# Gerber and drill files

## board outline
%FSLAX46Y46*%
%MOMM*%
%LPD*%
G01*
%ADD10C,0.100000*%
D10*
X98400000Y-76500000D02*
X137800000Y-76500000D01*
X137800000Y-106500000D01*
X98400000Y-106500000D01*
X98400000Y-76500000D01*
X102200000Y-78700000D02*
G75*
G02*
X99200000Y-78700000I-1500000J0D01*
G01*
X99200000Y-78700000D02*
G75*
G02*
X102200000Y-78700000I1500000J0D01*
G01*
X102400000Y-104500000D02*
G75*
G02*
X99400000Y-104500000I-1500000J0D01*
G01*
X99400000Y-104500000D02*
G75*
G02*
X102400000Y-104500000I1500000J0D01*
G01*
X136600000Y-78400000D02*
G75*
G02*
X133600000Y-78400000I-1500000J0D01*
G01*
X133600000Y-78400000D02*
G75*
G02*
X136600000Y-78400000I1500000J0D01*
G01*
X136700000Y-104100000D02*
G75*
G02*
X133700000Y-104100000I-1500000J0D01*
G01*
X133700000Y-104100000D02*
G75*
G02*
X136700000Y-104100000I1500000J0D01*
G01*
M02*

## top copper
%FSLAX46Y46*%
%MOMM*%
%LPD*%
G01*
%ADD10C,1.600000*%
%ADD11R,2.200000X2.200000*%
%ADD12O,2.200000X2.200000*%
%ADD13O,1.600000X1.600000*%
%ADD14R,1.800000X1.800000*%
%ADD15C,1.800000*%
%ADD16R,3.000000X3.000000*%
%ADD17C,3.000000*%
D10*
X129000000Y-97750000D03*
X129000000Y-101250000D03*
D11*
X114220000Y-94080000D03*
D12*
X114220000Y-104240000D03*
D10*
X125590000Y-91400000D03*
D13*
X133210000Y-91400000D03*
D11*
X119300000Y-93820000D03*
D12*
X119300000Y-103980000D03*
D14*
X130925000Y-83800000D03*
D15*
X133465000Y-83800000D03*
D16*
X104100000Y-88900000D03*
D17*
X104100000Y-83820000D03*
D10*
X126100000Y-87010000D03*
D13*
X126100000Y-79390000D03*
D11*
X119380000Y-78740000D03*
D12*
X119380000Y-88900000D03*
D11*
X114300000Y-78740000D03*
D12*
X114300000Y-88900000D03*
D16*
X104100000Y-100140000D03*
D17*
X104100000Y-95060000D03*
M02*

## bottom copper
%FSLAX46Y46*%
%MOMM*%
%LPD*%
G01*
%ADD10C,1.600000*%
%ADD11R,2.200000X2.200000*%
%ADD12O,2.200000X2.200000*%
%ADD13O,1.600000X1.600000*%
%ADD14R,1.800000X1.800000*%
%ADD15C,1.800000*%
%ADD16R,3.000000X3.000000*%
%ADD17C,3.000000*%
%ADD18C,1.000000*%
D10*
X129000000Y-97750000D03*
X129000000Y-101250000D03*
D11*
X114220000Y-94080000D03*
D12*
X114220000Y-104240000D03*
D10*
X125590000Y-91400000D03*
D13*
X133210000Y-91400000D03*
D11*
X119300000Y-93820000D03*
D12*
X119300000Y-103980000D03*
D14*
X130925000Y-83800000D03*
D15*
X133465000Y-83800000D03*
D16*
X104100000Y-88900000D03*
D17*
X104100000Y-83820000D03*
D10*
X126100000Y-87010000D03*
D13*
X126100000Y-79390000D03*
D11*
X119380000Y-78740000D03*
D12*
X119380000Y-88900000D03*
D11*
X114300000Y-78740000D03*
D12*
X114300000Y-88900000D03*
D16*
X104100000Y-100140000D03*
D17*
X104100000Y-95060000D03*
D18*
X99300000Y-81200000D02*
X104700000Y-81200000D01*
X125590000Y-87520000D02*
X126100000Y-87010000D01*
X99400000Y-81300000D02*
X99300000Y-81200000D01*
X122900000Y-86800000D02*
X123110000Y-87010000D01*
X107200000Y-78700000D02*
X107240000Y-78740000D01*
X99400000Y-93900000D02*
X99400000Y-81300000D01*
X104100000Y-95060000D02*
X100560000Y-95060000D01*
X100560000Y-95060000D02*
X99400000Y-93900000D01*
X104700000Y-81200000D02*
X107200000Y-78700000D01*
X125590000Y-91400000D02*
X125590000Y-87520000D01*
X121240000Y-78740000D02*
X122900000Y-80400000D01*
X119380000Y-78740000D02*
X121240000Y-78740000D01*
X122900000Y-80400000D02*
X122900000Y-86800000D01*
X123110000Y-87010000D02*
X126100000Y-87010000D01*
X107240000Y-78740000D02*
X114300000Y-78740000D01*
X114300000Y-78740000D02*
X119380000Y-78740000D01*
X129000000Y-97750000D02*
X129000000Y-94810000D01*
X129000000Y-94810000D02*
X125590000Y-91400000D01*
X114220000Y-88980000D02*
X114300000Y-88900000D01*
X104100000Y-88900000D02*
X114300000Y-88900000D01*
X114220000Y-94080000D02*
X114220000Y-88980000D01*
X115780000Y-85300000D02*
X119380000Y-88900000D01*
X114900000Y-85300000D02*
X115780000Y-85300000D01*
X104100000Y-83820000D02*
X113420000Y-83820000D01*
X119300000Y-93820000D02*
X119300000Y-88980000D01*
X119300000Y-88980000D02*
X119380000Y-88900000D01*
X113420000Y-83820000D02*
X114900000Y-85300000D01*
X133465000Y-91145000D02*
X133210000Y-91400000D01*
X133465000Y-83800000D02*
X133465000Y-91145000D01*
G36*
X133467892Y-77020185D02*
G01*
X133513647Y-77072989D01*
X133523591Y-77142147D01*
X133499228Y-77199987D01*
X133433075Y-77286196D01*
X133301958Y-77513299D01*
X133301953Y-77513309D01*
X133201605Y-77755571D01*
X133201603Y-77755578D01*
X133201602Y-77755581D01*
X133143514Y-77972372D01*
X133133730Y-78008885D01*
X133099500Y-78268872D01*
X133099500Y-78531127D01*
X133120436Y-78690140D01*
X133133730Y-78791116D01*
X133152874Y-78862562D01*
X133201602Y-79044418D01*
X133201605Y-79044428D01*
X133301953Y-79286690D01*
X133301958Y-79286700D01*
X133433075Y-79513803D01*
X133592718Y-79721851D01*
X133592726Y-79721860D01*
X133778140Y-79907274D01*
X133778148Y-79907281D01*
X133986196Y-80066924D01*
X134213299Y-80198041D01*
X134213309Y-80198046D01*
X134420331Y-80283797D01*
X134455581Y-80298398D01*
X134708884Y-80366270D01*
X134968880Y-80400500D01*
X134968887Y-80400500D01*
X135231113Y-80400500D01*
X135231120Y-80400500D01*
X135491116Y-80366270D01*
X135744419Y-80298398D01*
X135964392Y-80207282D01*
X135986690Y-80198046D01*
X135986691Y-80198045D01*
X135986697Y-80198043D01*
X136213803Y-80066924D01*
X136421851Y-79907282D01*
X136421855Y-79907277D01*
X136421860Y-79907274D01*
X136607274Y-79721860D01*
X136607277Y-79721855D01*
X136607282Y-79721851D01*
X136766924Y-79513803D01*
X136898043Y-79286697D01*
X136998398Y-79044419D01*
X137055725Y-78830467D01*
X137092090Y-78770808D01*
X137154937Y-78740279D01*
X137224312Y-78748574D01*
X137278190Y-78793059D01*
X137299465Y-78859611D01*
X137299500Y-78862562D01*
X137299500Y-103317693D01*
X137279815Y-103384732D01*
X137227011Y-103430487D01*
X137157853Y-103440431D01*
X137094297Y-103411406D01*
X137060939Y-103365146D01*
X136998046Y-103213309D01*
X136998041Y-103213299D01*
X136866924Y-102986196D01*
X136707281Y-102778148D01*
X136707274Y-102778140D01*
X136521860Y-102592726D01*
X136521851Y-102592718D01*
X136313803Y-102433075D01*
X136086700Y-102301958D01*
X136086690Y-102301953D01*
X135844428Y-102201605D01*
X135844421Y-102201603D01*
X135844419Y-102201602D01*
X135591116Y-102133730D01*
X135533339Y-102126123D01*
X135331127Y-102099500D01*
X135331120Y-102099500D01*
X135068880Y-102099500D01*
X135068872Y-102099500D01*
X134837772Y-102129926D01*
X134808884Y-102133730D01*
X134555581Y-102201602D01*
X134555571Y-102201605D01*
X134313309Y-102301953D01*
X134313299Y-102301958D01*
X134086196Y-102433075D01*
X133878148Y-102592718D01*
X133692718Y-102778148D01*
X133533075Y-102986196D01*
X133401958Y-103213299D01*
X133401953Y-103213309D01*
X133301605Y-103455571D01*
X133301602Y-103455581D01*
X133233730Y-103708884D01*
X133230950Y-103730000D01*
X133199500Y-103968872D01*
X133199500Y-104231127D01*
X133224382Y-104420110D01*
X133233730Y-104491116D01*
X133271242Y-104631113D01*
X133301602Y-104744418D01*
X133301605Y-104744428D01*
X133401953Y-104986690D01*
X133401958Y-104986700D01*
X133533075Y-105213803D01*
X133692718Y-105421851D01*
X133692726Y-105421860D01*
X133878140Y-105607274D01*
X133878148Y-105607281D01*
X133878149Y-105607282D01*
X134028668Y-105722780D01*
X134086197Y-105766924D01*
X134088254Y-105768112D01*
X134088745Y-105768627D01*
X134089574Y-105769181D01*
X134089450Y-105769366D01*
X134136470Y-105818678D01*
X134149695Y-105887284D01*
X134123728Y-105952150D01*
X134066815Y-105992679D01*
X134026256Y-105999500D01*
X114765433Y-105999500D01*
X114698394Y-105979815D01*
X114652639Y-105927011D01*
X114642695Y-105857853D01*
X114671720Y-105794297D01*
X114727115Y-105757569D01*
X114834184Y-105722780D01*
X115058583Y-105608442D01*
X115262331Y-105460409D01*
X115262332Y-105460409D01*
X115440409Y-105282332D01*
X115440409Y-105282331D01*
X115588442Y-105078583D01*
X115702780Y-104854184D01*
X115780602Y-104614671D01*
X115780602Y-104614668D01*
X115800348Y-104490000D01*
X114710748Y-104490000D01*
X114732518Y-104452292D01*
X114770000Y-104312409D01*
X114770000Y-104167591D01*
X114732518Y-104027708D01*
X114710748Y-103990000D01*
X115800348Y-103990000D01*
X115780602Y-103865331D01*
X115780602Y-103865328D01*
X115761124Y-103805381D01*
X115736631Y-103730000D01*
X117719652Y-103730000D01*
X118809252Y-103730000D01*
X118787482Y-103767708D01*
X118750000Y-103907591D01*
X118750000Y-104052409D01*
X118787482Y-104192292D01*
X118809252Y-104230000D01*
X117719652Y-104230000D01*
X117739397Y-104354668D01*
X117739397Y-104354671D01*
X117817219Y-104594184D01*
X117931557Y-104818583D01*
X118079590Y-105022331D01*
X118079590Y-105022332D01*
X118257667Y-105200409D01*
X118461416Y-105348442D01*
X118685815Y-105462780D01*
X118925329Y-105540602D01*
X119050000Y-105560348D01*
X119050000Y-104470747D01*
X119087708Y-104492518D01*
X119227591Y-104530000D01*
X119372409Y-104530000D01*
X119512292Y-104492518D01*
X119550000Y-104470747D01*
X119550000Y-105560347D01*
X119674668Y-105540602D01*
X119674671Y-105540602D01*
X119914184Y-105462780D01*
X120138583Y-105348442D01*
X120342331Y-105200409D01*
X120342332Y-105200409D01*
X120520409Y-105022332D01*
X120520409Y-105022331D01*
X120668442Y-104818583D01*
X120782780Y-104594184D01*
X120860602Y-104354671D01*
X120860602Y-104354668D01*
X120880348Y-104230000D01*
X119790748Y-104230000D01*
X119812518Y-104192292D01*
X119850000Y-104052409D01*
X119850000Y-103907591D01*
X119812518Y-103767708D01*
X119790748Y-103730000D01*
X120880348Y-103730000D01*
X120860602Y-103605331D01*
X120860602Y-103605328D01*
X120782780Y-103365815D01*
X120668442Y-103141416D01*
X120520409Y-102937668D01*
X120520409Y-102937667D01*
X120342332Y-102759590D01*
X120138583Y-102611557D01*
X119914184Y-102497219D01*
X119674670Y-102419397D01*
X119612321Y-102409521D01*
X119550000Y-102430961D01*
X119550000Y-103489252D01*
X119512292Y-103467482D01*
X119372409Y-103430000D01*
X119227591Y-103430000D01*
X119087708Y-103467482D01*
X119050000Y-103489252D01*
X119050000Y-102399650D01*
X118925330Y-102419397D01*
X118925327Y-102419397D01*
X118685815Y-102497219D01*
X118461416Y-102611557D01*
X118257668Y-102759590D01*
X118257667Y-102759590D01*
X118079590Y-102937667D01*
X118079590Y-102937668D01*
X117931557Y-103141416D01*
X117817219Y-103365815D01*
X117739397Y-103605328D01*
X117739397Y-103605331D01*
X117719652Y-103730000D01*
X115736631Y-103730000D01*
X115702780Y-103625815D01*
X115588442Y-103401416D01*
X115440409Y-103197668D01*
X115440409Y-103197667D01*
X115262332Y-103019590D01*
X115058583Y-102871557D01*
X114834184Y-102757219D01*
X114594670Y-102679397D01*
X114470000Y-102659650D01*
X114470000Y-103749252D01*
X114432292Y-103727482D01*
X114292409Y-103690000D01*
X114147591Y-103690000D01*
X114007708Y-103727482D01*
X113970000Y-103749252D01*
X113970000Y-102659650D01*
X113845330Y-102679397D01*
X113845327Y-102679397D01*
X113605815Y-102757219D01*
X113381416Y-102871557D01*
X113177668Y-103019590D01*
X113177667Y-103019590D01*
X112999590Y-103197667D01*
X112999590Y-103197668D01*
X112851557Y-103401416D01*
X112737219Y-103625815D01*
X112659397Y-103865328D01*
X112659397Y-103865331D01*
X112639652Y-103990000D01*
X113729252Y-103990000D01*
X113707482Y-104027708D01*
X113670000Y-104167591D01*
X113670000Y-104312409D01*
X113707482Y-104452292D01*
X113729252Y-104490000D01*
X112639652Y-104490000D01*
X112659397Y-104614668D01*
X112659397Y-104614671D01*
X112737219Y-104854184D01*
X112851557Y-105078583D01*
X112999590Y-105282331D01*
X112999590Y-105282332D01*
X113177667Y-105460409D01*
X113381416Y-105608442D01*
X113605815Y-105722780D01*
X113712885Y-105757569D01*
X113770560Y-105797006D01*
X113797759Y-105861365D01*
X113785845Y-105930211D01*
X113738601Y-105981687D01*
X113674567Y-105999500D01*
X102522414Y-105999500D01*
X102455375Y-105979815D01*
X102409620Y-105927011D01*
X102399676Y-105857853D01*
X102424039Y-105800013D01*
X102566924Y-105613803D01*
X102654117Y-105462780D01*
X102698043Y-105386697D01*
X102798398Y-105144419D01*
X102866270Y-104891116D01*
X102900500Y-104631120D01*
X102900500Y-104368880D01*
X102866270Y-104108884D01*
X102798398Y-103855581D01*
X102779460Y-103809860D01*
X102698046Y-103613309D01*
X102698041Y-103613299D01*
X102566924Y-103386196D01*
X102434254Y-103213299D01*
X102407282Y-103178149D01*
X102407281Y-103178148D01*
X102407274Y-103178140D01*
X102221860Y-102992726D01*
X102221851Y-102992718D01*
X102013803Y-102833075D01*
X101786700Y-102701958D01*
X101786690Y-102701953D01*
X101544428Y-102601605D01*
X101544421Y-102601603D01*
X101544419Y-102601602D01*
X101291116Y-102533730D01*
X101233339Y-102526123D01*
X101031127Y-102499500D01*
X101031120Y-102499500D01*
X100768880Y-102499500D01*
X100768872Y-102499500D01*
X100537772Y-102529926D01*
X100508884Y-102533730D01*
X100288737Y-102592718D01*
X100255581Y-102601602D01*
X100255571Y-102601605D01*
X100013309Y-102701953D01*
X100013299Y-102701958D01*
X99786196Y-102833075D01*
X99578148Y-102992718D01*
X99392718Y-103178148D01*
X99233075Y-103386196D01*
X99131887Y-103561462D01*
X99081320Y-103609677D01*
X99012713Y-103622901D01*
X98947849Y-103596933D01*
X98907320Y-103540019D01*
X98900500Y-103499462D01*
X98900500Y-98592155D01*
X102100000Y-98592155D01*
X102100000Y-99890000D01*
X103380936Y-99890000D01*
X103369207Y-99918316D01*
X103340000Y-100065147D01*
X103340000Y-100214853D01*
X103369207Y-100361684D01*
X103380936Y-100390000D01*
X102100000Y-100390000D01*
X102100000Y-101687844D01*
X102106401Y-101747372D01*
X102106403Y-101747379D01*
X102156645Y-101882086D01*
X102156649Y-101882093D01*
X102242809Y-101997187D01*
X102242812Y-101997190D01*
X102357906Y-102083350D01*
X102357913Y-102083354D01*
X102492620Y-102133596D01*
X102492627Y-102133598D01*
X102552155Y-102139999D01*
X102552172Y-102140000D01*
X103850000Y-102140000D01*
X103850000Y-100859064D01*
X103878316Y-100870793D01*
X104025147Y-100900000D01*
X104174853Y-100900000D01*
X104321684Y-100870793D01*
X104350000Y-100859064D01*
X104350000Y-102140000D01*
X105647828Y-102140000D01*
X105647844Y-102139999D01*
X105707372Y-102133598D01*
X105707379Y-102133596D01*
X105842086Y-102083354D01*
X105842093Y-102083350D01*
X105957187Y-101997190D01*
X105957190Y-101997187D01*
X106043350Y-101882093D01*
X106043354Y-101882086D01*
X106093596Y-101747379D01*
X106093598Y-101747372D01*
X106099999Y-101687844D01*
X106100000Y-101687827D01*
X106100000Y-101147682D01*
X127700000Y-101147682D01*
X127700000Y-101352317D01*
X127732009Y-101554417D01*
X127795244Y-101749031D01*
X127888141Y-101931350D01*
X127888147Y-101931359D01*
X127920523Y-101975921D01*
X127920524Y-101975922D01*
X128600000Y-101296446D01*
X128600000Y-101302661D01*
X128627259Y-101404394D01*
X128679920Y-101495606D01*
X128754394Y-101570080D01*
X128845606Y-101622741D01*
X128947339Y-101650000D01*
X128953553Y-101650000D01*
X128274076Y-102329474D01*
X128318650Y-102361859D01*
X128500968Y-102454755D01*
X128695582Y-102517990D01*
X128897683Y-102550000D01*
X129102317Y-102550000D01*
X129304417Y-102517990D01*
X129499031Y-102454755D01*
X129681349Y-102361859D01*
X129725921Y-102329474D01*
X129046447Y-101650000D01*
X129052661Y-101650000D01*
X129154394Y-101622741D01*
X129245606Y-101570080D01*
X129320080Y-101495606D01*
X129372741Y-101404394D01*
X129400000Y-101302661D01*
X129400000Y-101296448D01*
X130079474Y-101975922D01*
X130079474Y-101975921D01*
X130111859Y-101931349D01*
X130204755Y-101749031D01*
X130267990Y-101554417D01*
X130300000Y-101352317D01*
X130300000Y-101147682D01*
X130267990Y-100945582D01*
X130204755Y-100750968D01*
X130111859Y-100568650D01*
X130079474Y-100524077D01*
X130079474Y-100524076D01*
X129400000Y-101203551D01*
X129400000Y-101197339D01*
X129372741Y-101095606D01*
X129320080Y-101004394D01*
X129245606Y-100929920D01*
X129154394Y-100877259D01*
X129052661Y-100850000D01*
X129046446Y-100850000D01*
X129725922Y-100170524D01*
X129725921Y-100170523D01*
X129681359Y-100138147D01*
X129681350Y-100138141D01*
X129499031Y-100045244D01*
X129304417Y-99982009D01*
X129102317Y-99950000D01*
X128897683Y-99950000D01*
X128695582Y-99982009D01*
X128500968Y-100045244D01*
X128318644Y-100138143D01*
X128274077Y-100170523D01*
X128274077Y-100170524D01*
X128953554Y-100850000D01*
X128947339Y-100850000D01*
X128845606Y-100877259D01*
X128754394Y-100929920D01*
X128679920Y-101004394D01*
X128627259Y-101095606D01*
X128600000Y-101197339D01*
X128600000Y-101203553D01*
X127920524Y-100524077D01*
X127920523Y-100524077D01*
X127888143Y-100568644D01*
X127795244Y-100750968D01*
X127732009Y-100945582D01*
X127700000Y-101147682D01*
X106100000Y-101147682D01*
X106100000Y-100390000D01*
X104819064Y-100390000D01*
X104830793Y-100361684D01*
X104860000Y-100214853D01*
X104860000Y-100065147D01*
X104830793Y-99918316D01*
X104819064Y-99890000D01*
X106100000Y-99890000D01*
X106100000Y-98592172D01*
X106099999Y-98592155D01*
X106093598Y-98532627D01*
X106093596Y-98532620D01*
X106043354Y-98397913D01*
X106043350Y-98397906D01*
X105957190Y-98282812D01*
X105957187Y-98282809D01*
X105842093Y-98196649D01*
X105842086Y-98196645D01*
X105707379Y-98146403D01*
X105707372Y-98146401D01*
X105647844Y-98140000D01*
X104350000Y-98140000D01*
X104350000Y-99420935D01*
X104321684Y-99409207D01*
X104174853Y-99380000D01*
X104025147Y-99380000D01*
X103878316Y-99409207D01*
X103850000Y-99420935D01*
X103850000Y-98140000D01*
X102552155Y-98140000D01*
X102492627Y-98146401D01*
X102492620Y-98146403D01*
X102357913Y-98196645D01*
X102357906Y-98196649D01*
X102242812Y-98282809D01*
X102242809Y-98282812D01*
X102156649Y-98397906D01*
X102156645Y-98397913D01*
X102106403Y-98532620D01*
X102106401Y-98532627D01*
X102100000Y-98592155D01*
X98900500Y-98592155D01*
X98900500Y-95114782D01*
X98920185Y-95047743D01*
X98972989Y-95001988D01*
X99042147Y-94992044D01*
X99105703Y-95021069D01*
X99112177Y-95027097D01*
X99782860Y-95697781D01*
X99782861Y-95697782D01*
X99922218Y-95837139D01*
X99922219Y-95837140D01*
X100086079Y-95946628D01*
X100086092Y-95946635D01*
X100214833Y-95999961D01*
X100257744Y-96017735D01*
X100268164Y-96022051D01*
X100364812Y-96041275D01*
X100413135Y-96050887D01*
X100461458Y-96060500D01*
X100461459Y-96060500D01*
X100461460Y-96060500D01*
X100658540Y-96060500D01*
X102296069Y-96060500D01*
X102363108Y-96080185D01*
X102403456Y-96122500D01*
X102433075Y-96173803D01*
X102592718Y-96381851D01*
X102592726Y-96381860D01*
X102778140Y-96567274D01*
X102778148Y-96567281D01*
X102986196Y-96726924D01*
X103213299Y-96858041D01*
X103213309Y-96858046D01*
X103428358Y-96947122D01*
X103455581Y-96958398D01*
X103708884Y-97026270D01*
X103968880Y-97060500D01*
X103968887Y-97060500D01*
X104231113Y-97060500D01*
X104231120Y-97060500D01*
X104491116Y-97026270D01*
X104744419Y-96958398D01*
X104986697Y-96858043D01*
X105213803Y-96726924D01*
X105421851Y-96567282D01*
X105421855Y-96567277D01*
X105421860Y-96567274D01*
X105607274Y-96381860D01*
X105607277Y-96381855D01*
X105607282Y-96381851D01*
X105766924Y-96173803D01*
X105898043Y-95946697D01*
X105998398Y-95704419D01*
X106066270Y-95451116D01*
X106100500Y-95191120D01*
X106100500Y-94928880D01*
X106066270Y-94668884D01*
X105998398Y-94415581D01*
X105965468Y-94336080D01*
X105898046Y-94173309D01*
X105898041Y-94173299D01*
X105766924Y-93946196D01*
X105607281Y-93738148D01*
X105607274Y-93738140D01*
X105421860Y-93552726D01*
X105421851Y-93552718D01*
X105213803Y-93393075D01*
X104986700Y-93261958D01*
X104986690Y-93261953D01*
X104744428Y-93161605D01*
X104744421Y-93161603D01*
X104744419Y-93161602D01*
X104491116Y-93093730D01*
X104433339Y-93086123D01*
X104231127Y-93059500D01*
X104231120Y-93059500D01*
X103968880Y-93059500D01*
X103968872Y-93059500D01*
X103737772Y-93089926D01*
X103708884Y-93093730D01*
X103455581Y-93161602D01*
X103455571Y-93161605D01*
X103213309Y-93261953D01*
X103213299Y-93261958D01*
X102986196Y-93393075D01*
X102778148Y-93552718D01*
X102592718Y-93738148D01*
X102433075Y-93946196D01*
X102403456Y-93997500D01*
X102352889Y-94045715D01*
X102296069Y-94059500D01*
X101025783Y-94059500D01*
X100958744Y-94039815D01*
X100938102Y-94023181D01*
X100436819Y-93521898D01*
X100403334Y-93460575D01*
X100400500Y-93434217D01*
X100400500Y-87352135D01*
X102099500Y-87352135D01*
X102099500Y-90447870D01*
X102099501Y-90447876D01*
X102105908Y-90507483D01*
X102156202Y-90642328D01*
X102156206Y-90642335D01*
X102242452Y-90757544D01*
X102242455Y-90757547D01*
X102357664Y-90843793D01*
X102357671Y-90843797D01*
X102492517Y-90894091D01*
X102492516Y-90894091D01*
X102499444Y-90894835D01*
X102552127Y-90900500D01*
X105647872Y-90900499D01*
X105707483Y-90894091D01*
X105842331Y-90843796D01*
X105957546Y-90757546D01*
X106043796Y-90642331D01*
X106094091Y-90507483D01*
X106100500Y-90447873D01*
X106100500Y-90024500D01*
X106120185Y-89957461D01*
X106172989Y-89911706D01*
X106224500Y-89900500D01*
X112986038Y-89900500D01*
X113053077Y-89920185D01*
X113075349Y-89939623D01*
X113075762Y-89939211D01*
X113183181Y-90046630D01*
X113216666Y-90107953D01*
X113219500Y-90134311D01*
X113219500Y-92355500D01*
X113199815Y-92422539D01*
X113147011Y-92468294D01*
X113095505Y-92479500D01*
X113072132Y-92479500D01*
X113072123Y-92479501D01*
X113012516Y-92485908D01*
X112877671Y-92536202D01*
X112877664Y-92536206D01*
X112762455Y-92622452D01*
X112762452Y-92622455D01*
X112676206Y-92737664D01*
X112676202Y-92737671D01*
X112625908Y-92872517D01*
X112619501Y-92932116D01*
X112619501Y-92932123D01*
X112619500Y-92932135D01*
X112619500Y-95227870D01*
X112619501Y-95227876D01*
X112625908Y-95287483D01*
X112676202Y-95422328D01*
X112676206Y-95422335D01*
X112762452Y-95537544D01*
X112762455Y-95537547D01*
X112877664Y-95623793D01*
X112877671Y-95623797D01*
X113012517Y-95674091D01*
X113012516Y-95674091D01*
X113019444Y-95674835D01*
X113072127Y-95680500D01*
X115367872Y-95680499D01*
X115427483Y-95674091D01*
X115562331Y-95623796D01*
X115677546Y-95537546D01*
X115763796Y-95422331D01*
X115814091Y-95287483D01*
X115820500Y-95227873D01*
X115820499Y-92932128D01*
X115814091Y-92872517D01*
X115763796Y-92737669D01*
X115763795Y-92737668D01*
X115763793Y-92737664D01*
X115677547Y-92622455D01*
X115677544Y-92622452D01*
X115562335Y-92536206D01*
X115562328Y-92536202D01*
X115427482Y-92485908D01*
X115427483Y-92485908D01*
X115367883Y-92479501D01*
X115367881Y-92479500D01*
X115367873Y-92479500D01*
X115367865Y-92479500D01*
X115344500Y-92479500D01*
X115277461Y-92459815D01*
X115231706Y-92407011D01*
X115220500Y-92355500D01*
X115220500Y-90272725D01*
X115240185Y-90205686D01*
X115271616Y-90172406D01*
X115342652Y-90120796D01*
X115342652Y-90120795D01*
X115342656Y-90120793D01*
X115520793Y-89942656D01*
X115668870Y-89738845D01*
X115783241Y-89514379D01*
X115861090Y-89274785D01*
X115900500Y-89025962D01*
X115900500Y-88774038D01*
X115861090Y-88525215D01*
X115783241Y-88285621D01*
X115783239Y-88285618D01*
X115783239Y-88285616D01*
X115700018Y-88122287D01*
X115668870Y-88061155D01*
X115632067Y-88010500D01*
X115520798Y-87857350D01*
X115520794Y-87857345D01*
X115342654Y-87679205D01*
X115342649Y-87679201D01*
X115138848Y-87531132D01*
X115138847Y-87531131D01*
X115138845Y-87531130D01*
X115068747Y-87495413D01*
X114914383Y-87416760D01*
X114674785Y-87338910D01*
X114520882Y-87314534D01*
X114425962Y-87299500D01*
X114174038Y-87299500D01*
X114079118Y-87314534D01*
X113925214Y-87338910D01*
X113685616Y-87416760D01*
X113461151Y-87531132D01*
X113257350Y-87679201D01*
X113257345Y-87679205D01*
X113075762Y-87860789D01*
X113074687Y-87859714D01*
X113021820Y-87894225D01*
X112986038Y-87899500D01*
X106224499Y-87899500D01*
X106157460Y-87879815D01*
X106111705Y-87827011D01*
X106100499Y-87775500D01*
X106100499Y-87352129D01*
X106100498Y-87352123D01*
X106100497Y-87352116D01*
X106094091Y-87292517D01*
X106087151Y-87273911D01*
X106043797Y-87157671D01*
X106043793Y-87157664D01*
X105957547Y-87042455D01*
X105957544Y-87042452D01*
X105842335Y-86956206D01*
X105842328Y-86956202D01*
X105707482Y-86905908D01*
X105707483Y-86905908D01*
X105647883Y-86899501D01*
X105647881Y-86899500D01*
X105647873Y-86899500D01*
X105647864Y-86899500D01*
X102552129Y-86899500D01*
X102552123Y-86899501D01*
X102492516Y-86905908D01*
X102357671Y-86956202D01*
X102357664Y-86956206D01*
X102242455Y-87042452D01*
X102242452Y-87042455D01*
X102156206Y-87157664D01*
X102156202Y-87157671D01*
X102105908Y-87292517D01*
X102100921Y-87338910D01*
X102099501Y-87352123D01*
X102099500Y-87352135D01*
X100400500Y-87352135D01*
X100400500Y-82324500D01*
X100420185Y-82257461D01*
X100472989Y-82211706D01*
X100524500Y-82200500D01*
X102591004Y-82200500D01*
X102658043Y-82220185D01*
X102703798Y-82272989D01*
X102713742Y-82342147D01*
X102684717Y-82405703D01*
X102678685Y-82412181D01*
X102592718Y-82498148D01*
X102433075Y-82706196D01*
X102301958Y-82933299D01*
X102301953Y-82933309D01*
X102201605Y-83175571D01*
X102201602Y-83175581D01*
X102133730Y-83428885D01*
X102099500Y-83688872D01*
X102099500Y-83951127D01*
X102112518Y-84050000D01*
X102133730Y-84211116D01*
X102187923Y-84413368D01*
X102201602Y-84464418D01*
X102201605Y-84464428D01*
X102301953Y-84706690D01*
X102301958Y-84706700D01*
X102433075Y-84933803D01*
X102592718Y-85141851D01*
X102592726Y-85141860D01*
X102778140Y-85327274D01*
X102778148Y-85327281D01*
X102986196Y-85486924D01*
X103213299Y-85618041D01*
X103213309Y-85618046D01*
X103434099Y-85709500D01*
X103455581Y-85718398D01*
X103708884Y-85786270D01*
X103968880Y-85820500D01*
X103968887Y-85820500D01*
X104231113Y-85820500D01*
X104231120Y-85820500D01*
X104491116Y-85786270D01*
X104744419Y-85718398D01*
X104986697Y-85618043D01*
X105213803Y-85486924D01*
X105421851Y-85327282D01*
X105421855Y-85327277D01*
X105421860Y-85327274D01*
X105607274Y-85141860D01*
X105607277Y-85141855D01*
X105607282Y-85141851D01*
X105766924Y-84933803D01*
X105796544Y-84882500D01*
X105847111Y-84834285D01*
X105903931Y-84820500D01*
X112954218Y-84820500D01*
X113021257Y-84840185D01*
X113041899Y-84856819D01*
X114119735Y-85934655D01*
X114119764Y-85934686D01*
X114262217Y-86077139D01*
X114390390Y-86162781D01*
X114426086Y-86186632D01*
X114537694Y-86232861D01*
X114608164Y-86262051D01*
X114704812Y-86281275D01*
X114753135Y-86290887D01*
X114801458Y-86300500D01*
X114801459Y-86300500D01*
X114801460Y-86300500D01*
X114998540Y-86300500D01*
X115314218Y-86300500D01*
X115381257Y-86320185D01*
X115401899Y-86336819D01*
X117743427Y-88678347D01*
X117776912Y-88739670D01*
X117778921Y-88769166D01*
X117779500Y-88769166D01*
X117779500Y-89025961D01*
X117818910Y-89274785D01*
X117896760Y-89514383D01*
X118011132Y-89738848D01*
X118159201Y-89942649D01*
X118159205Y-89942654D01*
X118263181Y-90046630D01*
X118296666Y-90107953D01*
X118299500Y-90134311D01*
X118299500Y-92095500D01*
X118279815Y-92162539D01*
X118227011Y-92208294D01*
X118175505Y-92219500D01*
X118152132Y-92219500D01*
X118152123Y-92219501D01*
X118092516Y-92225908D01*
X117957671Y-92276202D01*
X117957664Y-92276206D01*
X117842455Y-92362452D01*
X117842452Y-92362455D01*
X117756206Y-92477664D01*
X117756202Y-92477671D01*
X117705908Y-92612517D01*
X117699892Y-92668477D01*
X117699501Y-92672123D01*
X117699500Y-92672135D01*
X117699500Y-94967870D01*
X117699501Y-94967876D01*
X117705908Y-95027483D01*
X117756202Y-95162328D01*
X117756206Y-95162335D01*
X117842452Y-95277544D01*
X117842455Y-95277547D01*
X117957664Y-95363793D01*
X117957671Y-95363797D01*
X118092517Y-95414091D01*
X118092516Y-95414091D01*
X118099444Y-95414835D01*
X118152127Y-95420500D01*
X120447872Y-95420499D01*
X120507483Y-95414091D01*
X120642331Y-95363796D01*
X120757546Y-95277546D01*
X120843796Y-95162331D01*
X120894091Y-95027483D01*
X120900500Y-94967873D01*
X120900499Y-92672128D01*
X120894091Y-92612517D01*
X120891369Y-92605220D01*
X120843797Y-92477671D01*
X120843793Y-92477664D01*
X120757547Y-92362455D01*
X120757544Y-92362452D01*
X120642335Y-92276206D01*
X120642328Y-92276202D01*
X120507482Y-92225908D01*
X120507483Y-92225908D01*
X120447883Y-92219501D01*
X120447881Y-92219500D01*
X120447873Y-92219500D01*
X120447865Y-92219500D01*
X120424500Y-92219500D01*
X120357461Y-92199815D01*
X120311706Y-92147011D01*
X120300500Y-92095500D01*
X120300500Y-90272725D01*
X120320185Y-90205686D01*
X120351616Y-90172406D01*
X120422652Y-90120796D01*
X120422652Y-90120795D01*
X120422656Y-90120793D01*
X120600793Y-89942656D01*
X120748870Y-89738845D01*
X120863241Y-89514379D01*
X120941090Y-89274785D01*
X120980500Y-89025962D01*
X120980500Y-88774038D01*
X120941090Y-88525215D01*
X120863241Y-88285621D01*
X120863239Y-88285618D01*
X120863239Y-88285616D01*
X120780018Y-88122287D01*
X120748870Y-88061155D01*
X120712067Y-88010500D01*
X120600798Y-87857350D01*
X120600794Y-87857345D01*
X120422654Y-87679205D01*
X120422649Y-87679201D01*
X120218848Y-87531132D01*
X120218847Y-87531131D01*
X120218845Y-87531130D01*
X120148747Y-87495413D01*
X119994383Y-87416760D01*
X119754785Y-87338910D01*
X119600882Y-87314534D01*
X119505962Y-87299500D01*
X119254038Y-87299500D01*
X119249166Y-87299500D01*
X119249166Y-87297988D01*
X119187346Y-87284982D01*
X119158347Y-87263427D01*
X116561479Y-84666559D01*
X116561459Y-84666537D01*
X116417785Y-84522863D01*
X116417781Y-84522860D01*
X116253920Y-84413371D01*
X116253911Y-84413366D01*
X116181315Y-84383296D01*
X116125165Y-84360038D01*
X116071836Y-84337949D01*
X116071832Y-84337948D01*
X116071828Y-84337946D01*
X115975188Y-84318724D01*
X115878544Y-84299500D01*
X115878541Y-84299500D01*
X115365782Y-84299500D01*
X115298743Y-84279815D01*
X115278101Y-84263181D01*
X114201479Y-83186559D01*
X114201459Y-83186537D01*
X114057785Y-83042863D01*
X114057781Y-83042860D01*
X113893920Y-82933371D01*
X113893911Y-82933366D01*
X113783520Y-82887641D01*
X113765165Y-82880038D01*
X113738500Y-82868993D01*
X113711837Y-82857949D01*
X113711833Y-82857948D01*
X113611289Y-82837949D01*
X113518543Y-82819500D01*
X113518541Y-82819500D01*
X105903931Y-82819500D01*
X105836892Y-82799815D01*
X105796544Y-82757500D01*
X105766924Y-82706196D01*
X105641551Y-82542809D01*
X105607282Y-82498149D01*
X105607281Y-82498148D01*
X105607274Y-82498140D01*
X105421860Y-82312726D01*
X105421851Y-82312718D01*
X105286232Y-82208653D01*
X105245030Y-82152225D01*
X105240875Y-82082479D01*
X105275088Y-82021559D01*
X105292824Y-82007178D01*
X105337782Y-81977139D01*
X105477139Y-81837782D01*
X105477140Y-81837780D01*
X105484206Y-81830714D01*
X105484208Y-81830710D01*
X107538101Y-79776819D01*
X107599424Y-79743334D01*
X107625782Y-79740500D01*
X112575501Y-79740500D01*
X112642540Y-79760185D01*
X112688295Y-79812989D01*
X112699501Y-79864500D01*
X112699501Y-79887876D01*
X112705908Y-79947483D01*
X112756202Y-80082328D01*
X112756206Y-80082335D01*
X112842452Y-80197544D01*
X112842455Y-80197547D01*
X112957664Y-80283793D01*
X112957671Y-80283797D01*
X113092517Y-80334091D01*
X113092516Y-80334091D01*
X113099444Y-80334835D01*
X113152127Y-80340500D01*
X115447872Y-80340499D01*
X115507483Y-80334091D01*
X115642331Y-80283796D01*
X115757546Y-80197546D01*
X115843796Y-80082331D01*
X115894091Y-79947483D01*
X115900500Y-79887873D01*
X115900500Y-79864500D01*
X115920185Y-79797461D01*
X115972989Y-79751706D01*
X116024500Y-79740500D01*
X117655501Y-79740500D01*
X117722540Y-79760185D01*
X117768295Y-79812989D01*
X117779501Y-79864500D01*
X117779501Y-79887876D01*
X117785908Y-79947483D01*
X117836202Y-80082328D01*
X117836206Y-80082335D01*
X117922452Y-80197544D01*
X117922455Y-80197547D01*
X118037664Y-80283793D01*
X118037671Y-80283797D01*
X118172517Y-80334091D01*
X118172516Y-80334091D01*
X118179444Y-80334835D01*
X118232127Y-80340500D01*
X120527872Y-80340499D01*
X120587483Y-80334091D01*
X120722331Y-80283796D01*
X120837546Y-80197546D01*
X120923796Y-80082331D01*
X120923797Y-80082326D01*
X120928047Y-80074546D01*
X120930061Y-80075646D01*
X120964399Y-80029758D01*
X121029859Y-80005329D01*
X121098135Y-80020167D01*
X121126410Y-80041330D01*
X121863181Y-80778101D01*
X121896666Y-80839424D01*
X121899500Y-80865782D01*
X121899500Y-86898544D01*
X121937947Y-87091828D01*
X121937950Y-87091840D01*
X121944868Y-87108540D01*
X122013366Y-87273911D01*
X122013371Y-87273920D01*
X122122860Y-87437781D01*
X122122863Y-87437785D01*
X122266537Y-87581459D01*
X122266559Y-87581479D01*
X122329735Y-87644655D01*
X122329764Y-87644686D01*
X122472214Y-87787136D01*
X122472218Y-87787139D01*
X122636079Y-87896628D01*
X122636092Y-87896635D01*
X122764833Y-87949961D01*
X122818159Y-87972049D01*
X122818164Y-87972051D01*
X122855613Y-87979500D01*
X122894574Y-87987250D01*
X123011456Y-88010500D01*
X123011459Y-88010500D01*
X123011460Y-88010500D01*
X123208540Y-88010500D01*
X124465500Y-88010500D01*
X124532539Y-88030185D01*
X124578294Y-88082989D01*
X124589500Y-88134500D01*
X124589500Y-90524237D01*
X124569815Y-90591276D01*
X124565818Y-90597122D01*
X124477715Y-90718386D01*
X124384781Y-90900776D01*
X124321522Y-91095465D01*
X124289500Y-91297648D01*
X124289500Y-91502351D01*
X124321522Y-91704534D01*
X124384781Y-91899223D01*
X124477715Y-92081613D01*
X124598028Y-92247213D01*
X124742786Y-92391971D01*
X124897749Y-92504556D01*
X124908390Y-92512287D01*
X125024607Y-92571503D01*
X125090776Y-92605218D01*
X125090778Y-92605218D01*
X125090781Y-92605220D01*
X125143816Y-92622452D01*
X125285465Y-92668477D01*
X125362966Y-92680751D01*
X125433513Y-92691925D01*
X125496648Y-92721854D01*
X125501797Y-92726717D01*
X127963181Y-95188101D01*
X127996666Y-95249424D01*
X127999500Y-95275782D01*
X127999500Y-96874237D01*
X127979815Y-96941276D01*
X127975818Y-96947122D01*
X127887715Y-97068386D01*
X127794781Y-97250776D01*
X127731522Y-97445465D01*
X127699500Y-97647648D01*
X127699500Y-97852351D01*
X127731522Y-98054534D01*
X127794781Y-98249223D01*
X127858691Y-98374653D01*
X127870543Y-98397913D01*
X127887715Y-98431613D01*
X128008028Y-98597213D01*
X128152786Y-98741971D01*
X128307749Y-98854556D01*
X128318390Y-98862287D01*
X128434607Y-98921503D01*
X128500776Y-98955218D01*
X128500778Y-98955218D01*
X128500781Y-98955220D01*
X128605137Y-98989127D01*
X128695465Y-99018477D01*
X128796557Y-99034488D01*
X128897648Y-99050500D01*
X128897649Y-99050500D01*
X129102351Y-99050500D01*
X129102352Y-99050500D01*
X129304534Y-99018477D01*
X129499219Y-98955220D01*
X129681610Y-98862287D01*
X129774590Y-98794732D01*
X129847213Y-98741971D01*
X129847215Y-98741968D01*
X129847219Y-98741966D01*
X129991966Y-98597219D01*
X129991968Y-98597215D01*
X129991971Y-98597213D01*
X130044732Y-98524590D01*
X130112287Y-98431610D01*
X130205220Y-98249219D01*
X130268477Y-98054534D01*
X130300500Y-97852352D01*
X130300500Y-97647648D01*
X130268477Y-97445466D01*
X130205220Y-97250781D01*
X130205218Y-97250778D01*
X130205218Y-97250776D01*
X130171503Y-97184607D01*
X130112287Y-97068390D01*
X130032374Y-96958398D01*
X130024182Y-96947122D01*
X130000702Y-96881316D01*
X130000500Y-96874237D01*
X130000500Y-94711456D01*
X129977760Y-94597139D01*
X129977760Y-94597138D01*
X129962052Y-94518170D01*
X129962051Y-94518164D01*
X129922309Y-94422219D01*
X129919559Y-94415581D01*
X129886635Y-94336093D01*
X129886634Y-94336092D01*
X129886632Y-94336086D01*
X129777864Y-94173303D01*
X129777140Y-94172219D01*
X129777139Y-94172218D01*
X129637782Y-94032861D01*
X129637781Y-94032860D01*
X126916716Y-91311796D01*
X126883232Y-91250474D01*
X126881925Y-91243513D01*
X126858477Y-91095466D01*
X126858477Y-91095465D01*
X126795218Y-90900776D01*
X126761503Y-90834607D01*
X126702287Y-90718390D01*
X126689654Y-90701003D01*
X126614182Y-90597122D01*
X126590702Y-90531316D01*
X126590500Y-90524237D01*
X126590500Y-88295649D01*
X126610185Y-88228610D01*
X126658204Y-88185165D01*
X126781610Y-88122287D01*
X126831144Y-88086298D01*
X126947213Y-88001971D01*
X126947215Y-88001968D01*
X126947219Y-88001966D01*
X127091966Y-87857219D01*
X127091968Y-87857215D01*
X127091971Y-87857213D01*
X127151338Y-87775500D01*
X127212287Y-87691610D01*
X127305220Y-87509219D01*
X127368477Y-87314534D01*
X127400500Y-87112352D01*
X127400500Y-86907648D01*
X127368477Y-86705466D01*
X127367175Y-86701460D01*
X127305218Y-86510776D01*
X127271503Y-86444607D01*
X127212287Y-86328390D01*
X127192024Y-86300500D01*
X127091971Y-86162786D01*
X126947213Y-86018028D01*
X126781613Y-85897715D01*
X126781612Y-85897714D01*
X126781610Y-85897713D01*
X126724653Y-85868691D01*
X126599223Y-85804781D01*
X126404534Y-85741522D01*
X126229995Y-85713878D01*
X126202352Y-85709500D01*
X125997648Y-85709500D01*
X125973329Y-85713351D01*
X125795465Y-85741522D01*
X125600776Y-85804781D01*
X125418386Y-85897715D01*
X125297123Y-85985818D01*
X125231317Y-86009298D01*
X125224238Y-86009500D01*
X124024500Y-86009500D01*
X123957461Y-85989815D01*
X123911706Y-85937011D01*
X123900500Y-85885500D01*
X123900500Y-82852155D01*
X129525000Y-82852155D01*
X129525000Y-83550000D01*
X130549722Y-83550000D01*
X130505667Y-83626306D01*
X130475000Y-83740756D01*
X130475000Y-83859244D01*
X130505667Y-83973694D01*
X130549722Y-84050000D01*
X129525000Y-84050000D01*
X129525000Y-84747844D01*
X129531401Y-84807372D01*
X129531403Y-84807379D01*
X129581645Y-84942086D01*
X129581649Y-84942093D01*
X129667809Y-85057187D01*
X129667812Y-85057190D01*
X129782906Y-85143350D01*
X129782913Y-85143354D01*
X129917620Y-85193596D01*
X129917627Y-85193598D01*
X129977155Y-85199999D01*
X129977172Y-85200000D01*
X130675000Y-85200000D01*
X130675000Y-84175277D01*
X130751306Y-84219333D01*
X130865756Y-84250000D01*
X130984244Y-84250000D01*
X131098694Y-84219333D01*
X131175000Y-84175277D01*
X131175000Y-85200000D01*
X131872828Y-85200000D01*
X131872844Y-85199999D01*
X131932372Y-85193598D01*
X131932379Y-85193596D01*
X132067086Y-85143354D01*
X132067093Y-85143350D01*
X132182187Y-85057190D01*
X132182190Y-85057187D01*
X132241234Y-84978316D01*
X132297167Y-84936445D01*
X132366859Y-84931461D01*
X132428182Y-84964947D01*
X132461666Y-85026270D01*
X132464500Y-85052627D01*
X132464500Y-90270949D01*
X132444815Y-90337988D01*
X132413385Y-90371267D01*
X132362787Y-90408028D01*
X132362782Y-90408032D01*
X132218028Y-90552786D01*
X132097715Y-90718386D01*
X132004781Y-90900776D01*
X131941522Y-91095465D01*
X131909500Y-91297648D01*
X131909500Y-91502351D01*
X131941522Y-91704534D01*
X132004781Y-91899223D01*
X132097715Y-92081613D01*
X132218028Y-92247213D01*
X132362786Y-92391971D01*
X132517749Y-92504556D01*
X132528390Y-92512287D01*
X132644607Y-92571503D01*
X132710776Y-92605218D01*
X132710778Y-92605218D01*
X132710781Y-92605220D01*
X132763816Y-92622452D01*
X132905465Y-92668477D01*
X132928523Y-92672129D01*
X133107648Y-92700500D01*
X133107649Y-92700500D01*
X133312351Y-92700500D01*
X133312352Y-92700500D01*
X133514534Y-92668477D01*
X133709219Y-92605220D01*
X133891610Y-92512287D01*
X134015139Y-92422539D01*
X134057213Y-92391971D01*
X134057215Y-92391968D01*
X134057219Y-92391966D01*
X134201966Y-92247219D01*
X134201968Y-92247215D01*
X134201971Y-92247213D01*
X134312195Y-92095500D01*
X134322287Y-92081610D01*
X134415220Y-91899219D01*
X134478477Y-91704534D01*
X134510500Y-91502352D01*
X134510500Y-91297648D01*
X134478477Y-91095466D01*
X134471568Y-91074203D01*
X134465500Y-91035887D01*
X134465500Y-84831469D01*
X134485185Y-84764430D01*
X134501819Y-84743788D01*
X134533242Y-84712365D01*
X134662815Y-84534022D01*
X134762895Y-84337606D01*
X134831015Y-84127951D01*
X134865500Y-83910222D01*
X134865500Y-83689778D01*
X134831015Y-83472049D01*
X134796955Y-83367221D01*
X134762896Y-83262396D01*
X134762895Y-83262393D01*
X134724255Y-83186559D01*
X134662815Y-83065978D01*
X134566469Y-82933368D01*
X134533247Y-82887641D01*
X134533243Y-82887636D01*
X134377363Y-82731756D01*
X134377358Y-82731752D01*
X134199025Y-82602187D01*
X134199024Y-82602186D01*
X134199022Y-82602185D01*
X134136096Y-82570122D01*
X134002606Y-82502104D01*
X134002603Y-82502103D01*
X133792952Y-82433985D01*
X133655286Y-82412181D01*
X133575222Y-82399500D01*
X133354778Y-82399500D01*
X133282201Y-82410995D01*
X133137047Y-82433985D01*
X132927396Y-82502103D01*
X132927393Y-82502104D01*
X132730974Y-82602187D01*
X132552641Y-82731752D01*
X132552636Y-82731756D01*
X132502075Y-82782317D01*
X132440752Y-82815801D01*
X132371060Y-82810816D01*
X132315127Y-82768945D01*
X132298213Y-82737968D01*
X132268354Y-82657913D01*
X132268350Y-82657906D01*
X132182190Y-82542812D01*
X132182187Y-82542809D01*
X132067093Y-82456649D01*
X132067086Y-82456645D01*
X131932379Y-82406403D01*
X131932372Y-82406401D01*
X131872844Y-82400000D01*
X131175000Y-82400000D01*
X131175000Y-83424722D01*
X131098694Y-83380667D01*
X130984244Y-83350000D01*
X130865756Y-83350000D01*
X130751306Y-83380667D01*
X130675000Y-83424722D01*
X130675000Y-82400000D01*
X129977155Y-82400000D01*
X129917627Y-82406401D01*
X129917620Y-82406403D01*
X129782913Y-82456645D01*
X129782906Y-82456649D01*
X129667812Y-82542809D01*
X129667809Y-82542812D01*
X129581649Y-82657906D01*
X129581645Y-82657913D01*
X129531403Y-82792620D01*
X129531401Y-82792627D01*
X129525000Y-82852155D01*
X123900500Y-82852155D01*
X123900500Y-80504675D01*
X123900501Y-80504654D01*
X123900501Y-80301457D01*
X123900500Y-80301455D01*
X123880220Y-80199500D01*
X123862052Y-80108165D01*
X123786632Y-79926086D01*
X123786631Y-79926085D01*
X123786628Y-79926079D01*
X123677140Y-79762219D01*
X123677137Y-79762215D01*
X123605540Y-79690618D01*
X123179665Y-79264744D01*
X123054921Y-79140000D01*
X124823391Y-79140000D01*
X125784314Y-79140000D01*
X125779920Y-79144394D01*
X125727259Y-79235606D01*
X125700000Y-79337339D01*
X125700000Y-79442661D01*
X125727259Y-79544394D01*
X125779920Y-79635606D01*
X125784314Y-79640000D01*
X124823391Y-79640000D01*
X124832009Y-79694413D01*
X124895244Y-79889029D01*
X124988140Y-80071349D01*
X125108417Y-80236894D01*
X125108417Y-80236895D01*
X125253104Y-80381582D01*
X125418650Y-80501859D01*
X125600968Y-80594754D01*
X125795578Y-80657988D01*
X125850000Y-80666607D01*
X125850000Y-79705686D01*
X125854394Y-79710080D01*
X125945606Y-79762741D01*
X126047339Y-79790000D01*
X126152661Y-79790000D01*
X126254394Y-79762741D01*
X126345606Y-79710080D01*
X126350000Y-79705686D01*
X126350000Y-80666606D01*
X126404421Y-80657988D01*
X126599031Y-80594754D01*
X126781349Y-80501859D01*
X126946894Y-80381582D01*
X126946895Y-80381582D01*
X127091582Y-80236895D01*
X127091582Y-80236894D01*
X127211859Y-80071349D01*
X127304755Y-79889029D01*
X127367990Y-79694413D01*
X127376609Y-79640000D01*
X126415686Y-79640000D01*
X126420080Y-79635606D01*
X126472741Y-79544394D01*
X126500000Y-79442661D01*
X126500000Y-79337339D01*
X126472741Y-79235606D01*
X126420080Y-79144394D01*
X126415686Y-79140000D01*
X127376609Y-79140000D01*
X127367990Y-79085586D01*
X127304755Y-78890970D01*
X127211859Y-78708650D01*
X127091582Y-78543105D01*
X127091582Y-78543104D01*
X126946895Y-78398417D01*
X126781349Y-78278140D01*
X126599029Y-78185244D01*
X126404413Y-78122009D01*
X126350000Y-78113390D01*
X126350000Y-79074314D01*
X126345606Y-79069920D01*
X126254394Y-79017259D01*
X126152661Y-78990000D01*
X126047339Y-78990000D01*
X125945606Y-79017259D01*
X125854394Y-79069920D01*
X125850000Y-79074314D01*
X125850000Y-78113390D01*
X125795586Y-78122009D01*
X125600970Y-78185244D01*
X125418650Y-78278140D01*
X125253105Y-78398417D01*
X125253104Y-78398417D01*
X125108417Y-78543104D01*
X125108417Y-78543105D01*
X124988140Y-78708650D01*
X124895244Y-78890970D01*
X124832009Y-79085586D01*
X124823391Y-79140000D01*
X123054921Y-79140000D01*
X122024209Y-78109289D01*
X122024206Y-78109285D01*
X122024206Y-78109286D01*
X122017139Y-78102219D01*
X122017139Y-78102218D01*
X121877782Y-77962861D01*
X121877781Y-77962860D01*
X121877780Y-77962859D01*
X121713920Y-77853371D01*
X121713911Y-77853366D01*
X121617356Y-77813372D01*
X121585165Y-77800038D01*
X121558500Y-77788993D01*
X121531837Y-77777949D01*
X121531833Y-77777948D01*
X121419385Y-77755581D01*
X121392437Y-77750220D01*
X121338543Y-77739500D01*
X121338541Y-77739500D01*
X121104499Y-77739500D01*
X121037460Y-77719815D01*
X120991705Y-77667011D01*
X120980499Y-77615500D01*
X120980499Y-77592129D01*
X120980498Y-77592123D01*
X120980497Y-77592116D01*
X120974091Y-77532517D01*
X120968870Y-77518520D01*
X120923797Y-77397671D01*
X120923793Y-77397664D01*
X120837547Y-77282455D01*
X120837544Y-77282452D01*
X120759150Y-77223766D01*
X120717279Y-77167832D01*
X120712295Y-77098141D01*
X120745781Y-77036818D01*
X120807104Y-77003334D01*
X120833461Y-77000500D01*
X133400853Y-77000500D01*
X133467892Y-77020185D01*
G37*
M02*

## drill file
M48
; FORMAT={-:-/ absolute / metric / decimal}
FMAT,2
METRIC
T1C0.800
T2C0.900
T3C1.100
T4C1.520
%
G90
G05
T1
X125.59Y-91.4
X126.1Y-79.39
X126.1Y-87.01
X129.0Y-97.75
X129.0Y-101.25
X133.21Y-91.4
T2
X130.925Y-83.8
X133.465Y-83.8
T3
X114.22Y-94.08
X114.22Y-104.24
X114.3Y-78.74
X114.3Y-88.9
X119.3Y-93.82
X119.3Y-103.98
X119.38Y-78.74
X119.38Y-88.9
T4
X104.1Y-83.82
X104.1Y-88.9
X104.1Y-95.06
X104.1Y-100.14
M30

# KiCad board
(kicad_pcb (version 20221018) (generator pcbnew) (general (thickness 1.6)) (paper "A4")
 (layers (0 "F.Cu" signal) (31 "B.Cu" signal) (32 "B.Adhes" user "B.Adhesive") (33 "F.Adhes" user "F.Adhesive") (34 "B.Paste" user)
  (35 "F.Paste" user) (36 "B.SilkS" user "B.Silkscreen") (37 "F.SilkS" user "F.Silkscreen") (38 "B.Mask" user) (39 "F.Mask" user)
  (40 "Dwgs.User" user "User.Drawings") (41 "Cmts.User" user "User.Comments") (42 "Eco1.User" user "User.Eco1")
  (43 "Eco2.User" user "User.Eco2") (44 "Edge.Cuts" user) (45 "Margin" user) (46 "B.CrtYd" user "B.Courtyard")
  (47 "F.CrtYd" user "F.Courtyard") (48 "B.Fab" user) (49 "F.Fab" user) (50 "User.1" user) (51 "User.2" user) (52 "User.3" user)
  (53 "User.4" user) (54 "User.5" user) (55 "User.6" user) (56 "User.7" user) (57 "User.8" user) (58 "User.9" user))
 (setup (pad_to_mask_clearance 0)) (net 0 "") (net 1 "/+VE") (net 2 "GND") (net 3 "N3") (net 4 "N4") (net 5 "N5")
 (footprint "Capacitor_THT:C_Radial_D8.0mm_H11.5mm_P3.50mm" (layer "F.Cu") (at 129 97.75 -90)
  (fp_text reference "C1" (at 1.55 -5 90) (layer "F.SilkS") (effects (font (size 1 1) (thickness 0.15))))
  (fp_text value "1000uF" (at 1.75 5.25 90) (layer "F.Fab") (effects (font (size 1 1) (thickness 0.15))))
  (pad "1" thru_hole circle (at 0 0 270) (size 1.6 1.6) (drill 0.8) (layers "*.Cu" "*.Mask") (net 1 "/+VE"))
  (pad "2" thru_hole circle (at 3.5 0 270) (size 1.6 1.6) (drill 0.8) (layers "*.Cu" "*.Mask") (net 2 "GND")))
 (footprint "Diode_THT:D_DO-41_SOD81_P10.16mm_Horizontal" (layer "F.Cu") (at 114.22 94.08 -90)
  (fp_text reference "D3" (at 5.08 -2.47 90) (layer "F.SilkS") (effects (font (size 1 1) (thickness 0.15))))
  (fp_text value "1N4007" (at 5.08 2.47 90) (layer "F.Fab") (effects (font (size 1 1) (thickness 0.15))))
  (pad "1" thru_hole rect (at 0 0 270) (size 2.2 2.2) (drill 1.1) (layers "*.Cu" "*.Mask") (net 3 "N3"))
  (pad "2" thru_hole oval (at 10.16 0 270) (size 2.2 2.2) (drill 1.1) (layers "*.Cu" "*.Mask") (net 2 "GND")))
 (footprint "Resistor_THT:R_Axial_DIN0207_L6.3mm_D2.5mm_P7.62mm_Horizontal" (layer "F.Cu") (at 125.59 91.4)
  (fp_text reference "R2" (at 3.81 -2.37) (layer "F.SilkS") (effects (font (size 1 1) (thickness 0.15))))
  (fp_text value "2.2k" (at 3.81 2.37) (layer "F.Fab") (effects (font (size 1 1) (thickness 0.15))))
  (pad "1" thru_hole circle (at 0 0) (size 1.6 1.6) (drill 0.8) (layers "*.Cu" "*.Mask") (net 1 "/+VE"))
  (pad "2" thru_hole oval (at 7.62 0) (size 1.6 1.6) (drill 0.8) (layers "*.Cu" "*.Mask") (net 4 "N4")))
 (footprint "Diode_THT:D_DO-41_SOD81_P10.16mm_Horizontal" (layer "F.Cu") (at 119.3 93.82 -90)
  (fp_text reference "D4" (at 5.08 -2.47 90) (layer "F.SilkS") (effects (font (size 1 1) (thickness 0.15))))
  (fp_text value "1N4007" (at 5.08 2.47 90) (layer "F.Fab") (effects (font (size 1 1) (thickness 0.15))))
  (pad "1" thru_hole rect (at 0 0 270) (size 2.2 2.2) (drill 1.1) (layers "*.Cu" "*.Mask") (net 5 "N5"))
  (pad "2" thru_hole oval (at 10.16 0 270) (size 2.2 2.2) (drill 1.1) (layers "*.Cu" "*.Mask") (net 2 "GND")))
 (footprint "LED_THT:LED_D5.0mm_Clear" (layer "F.Cu") (at 130.925 83.8)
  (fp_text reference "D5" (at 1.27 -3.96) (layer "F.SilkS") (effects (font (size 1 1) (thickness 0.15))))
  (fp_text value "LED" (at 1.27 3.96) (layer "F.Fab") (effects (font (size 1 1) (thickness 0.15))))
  (pad "1" thru_hole rect (at 0 0) (size 1.8 1.8) (drill 0.9) (layers "*.Cu" "*.Mask") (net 2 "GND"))
  (pad "2" thru_hole circle (at 2.54 0) (size 1.8 1.8) (drill 0.9) (layers "*.Cu" "*.Mask") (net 4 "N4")))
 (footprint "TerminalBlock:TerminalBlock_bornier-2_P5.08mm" (layer "F.Cu") (at 104.1 88.9 90)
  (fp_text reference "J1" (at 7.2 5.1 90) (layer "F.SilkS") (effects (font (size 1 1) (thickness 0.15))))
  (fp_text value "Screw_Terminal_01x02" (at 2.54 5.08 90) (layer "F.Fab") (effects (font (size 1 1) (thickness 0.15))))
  (pad "1" thru_hole rect (at 0 0 90) (size 3 3) (drill 1.52) (layers "*.Cu" "*.Mask") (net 3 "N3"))
  (pad "2" thru_hole circle (at 5.08 0 90) (size 3 3) (drill 1.52) (layers "*.Cu" "*.Mask") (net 5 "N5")))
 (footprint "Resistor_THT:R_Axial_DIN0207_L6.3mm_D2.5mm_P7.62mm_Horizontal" (layer "F.Cu") (at 126.1 87.01 90)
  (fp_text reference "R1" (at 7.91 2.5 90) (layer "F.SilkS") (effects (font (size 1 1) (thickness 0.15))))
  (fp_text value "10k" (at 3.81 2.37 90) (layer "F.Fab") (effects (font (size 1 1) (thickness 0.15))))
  (pad "1" thru_hole circle (at 0 0 90) (size 1.6 1.6) (drill 0.8) (layers "*.Cu" "*.Mask") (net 1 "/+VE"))
  (pad "2" thru_hole oval (at 7.62 0 90) (size 1.6 1.6) (drill 0.8) (layers "*.Cu" "*.Mask") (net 2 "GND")))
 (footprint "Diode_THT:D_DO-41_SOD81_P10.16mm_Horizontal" (layer "F.Cu") (at 119.38 78.74 -90)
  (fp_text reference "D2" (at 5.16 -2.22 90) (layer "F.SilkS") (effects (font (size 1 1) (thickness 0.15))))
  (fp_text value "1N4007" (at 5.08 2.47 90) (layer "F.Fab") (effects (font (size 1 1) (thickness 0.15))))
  (pad "1" thru_hole rect (at 0 0 270) (size 2.2 2.2) (drill 1.1) (layers "*.Cu" "*.Mask") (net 1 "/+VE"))
  (pad "2" thru_hole oval (at 10.16 0 270) (size 2.2 2.2) (drill 1.1) (layers "*.Cu" "*.Mask") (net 5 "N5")))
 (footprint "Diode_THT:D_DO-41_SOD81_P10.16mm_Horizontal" (layer "F.Cu") (at 114.3 78.74 -90)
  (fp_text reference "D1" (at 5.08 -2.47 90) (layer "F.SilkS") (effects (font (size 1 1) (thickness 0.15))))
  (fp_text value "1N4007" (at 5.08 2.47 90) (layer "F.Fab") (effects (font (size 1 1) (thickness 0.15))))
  (pad "1" thru_hole rect (at 0 0 270) (size 2.2 2.2) (drill 1.1) (layers "*.Cu" "*.Mask") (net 1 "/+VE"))
  (pad "2" thru_hole oval (at 10.16 0 270) (size 2.2 2.2) (drill 1.1) (layers "*.Cu" "*.Mask") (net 3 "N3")))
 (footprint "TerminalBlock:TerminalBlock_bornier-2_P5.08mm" (layer "F.Cu") (at 104.1 100.14 90)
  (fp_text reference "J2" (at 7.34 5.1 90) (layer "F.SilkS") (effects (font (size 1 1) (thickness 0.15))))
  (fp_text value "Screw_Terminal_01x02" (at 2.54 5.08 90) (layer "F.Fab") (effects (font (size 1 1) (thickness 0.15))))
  (pad "1" thru_hole rect (at 0 0 90) (size 3 3) (drill 1.52) (layers "*.Cu" "*.Mask") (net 2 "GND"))
  (pad "2" thru_hole circle (at 5.08 0 90) (size 3 3) (drill 1.52) (layers "*.Cu" "*.Mask") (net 1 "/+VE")))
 (gr_rect (start 98.4 76.5) (end 137.8 106.5) (stroke (width 0.1) (type default)) (fill none) (layer "Edge.Cuts"))
 (gr_circle (center 100.7 78.7) (end 99.8 79.9) (stroke (width 0.1) (type default)) (fill none) (layer "Edge.Cuts"))
 (gr_circle (center 100.9 104.5) (end 100 105.7) (stroke (width 0.1) (type default)) (fill none) (layer "Edge.Cuts"))
 (gr_circle (center 135.1 78.4) (end 134.2 79.6) (stroke (width 0.1) (type default)) (fill none) (layer "Edge.Cuts"))
 (gr_circle (center 135.2 104.1) (end 134.3 105.3) (stroke (width 0.1) (type default)) (fill none) (layer "Edge.Cuts"))
 (segment (start 99.3 81.2) (end 104.7 81.2) (width 1) (layer "B.Cu") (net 1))
 (segment (start 125.59 87.52) (end 126.1 87.01) (width 1) (layer "B.Cu") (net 1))
 (segment (start 99.4 81.3) (end 99.3 81.2) (width 1) (layer "B.Cu") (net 1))
 (segment (start 122.9 86.8) (end 123.11 87.01) (width 1) (layer "B.Cu") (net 1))
 (segment (start 107.2 78.7) (end 107.24 78.74) (width 1) (layer "B.Cu") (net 1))
 (segment (start 99.4 93.9) (end 99.4 81.3) (width 1) (layer "B.Cu") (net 1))
 (segment (start 104.1 95.06) (end 100.56 95.06) (width 1) (layer "B.Cu") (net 1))
 (segment (start 100.56 95.06) (end 99.4 93.9) (width 1) (layer "B.Cu") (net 1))
 (segment (start 104.7 81.2) (end 107.2 78.7) (width 1) (layer "B.Cu") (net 1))
 (segment (start 125.59 91.4) (end 125.59 87.52) (width 1) (layer "B.Cu") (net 1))
 (segment (start 121.24 78.74) (end 122.9 80.4) (width 1) (layer "B.Cu") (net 1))
 (segment (start 119.38 78.74) (end 121.24 78.74) (width 1) (layer "B.Cu") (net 1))
 (segment (start 122.9 80.4) (end 122.9 86.8) (width 1) (layer "B.Cu") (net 1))
 (segment (start 123.11 87.01) (end 126.1 87.01) (width 1) (layer "B.Cu") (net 1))
 (segment (start 107.24 78.74) (end 114.3 78.74) (width 1) (layer "B.Cu") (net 1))
 (segment (start 114.3 78.74) (end 119.38 78.74) (width 1) (layer "B.Cu") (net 1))
 (segment (start 129 97.75) (end 129 94.81) (width 1) (layer "B.Cu") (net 1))
 (segment (start 129 94.81) (end 125.59 91.4) (width 1) (layer "B.Cu") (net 1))
 (segment (start 114.22 88.98) (end 114.3 88.9) (width 1) (layer "B.Cu") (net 3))
 (segment (start 104.1 88.9) (end 114.3 88.9) (width 1) (layer "B.Cu") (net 3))
 (segment (start 114.22 94.08) (end 114.22 88.98) (width 1) (layer "B.Cu") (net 3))
 (segment (start 115.78 85.3) (end 119.38 88.9) (width 1) (layer "B.Cu") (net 5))
 (segment (start 114.9 85.3) (end 115.78 85.3) (width 1) (layer "B.Cu") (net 5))
 (segment (start 104.1 83.82) (end 113.42 83.82) (width 1) (layer "B.Cu") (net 5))
 (segment (start 119.3 93.82) (end 119.3 88.98) (width 1) (layer "B.Cu") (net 5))
 (segment (start 119.3 88.98) (end 119.38 88.9) (width 1) (layer "B.Cu") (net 5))
 (segment (start 113.42 83.82) (end 114.9 85.3) (width 1) (layer "B.Cu") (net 5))
 (segment (start 133.465 91.145) (end 133.21 91.4) (width 1) (layer "B.Cu") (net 4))
 (segment (start 133.465 83.8) (end 133.465 91.145) (width 1) (layer "B.Cu") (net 4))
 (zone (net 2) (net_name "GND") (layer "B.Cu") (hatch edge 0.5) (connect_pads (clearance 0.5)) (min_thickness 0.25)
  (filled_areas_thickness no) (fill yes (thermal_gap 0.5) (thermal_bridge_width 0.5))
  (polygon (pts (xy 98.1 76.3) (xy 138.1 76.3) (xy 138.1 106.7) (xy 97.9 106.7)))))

